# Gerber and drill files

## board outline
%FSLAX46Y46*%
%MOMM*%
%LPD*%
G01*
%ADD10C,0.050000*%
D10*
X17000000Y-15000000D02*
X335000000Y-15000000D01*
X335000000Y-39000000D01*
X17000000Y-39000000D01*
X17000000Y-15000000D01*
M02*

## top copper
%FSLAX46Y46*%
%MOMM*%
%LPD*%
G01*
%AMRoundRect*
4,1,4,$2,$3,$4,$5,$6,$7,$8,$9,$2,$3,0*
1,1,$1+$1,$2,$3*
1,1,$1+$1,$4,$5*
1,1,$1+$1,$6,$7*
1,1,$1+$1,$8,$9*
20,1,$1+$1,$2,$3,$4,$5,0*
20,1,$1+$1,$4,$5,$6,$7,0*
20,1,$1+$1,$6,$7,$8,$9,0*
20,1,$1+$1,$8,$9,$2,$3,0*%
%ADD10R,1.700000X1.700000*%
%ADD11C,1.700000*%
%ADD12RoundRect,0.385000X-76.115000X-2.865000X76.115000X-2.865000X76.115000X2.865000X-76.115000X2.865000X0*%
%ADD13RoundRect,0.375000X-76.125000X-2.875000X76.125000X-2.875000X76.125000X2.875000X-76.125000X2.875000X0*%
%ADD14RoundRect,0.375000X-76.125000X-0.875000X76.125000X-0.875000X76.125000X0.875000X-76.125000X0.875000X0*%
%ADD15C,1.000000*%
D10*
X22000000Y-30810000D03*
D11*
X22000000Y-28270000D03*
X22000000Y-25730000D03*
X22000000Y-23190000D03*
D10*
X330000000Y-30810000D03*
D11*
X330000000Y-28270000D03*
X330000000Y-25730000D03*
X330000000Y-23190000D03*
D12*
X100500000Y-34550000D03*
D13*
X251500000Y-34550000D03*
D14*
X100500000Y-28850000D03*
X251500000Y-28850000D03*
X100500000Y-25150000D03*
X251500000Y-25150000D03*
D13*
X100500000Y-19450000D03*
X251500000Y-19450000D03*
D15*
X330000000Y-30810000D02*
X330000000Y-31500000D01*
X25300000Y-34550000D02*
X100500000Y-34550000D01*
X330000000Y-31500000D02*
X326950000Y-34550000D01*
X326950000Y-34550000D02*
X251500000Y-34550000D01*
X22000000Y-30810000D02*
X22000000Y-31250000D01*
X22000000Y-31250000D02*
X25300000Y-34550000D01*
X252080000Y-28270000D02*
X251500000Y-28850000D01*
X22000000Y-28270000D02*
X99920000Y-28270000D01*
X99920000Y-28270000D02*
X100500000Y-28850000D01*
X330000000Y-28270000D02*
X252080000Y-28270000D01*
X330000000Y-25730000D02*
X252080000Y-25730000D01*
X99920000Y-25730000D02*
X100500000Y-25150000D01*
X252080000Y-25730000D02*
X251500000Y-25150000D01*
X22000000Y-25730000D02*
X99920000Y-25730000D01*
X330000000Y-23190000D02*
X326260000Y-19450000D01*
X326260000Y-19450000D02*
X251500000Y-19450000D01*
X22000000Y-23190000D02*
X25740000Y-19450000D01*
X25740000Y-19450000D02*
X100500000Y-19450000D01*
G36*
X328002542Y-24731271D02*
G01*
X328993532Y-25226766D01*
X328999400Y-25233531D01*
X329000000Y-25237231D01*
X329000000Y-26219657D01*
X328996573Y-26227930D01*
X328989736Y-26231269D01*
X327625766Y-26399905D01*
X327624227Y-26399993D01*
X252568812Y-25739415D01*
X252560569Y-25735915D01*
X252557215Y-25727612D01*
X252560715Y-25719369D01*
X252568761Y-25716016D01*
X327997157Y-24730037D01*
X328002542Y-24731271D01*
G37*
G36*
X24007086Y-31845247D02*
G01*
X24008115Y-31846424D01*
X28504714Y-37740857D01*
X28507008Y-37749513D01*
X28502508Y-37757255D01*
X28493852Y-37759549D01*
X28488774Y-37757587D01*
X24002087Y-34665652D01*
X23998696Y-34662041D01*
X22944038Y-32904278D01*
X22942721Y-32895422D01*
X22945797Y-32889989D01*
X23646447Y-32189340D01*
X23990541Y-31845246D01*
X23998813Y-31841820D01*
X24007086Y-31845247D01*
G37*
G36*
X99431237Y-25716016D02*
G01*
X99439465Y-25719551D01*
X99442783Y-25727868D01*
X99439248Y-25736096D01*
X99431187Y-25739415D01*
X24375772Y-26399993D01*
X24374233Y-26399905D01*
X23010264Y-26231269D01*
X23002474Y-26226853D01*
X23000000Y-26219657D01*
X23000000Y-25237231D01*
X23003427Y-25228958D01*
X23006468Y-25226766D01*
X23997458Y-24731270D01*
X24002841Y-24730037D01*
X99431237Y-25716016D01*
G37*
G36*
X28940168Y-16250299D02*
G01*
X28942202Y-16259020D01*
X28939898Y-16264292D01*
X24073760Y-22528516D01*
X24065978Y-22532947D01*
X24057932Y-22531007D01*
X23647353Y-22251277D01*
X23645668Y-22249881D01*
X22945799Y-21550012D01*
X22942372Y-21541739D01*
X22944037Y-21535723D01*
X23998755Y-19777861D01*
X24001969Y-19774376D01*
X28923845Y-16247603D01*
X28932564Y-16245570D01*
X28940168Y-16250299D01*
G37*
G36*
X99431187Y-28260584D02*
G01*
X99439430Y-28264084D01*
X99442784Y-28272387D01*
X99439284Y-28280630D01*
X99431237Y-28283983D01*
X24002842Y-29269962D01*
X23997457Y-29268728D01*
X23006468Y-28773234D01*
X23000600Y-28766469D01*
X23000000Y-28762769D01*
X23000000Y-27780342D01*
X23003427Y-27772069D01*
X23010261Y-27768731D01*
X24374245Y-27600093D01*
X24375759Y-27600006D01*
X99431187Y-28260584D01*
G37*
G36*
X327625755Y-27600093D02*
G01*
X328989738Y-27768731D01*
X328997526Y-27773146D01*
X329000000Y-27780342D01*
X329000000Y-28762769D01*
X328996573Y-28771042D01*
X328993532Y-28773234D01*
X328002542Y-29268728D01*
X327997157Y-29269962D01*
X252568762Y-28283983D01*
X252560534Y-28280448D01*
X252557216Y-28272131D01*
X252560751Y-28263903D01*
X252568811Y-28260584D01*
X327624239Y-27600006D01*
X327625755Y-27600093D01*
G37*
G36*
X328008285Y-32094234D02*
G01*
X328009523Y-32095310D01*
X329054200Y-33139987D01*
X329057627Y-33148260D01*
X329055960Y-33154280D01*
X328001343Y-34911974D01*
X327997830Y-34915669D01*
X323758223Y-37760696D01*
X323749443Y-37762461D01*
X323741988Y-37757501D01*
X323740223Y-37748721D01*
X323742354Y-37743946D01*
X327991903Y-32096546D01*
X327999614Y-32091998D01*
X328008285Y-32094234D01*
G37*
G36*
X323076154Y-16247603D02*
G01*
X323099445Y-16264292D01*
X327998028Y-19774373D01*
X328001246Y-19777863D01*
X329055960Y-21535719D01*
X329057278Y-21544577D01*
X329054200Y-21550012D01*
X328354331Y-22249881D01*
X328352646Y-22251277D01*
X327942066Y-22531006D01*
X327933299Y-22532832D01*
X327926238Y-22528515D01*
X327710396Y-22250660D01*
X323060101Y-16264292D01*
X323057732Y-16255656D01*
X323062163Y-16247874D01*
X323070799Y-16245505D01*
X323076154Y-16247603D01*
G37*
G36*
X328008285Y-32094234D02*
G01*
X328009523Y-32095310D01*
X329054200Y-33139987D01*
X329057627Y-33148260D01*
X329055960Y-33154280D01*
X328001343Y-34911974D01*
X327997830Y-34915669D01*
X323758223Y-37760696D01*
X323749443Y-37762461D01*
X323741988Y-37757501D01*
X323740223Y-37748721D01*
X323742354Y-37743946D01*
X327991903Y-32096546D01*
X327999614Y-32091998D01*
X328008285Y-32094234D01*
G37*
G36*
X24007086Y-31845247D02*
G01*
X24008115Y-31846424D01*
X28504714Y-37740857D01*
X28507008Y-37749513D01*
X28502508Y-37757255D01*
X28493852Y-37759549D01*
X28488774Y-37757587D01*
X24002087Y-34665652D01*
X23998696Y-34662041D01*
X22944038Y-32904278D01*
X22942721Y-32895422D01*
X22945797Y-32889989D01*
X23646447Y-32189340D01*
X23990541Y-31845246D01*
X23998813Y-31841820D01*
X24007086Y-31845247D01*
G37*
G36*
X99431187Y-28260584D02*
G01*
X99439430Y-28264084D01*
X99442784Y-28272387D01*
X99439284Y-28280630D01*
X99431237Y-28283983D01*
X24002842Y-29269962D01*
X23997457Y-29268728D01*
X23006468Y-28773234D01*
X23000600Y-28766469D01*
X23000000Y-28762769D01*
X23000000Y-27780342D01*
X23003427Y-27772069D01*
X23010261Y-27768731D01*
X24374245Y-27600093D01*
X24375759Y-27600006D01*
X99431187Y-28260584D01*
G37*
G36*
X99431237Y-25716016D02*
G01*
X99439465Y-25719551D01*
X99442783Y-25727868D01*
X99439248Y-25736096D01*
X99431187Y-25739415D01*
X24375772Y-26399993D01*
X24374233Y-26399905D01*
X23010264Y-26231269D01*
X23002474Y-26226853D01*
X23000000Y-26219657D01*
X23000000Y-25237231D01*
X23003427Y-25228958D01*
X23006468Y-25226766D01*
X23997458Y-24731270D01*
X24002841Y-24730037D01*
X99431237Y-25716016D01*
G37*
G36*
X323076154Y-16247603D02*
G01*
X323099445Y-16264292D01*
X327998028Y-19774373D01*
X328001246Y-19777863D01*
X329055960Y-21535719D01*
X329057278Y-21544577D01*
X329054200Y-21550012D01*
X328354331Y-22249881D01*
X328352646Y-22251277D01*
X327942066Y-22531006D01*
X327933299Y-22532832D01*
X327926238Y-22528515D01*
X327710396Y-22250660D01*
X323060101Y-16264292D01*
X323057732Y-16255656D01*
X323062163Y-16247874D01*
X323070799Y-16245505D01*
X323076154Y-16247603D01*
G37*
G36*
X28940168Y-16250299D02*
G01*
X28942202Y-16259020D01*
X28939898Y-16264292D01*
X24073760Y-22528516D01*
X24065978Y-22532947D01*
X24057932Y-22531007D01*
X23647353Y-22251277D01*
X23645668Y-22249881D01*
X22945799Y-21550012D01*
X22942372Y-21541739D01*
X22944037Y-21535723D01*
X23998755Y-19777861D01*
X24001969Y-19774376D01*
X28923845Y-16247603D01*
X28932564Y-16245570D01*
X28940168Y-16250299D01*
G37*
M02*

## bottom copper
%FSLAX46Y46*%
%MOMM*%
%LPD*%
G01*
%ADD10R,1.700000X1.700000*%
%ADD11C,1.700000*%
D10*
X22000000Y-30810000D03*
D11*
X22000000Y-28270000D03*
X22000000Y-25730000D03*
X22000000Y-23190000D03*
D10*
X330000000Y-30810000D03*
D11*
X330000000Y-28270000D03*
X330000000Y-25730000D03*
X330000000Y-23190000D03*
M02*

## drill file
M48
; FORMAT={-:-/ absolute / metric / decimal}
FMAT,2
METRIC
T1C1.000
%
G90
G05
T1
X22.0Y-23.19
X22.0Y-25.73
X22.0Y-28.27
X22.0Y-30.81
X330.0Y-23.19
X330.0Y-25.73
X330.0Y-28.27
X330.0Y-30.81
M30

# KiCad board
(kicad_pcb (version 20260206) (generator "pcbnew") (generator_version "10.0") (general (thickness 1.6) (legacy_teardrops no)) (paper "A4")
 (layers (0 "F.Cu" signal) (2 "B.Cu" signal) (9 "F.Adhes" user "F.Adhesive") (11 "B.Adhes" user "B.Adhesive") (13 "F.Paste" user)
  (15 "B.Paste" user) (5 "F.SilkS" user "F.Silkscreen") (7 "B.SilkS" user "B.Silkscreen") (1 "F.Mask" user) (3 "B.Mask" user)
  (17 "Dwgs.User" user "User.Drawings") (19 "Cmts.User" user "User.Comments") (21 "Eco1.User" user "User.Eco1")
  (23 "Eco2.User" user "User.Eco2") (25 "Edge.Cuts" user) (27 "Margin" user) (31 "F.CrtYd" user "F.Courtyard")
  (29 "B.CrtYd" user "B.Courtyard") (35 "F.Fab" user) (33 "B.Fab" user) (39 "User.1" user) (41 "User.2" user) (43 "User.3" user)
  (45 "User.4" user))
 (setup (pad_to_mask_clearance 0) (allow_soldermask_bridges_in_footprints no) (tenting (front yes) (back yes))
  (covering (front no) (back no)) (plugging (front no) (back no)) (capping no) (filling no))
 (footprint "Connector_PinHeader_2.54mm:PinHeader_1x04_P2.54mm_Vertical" (layer "F.Cu") (at 22 30.81 180)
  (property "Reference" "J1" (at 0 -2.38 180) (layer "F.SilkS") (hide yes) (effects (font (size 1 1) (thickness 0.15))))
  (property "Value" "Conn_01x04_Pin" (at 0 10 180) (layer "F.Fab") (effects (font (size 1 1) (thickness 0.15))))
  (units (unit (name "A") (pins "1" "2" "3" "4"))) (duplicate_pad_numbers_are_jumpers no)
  (pad "1" thru_hole rect (at 0 0 180) (size 1.7 1.7) (drill 1) (layers "*.Cu" "*.Mask") (remove_unused_layers no) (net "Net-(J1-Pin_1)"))
  (pad "2" thru_hole circle (at 0 2.54 180) (size 1.7 1.7) (drill 1) (layers "*.Cu" "*.Mask") (remove_unused_layers no)
   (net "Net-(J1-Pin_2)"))
  (pad "3" thru_hole circle (at 0 5.08 180) (size 1.7 1.7) (drill 1) (layers "*.Cu" "*.Mask") (remove_unused_layers no)
   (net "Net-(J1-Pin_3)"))
  (pad "4" thru_hole circle (at 0 7.62 180) (size 1.7 1.7) (drill 1) (layers "*.Cu" "*.Mask") (remove_unused_layers no)
   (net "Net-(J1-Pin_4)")))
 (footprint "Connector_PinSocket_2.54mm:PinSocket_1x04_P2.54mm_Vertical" (layer "F.Cu") (at 330 30.81 180)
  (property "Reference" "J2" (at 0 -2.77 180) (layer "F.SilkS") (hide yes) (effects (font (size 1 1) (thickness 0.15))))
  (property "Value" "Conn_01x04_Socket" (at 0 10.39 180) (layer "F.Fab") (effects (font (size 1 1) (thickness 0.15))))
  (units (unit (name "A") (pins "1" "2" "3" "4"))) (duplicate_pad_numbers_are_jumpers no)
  (pad "1" thru_hole rect (at 0 0 180) (size 1.7 1.7) (drill 1) (layers "*.Cu" "*.Mask") (remove_unused_layers no) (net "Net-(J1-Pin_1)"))
  (pad "2" thru_hole circle (at 0 2.54 180) (size 1.7 1.7) (drill 1) (layers "*.Cu" "*.Mask") (remove_unused_layers no)
   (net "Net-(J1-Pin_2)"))
  (pad "3" thru_hole circle (at 0 5.08 180) (size 1.7 1.7) (drill 1) (layers "*.Cu" "*.Mask") (remove_unused_layers no)
   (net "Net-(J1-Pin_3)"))
  (pad "4" thru_hole circle (at 0 7.62 180) (size 1.7 1.7) (drill 1) (layers "*.Cu" "*.Mask") (remove_unused_layers no)
   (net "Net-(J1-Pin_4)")))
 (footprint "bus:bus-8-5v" (layer "F.Cu") (at 23 15)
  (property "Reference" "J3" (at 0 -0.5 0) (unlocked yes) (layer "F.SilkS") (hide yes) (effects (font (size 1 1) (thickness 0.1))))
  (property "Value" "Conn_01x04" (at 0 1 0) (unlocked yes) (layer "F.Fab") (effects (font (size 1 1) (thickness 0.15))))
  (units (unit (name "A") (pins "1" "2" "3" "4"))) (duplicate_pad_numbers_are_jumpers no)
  (pad "1" smd roundrect (at 77.5 19.55) (size 153 6.5) (layers "F.Cu" "F.Mask" "F.Paste") (roundrect_rratio 0.05923076923)
   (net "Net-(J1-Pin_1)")
   (teardrops (best_length_ratio 0.5) (max_length 1) (best_width_ratio 1) (max_width 2) (curved_edges no) (filter_ratio 0.9) (enabled yes)
    (allow_two_segments yes) (prefer_zone_connections yes)))
  (pad "1" smd roundrect (at 228.5 19.55) (size 153 6.5) (layers "F.Cu" "F.Mask" "F.Paste") (roundrect_rratio 0.05769230769)
   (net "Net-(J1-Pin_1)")
   (teardrops (best_length_ratio 0.5) (max_length 1) (best_width_ratio 1) (max_width 2) (curved_edges no) (filter_ratio 0.9) (enabled yes)
    (allow_two_segments yes) (prefer_zone_connections yes)))
  (pad "2" smd roundrect (at 77.5 13.85) (size 153 2.5) (layers "F.Cu" "F.Mask" "F.Paste") (roundrect_rratio 0.15) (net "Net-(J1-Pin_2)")
   (teardrops (best_length_ratio 0.5) (max_length 1) (best_width_ratio 1) (max_width 2) (curved_edges no) (filter_ratio 0.9) (enabled yes)
    (allow_two_segments yes) (prefer_zone_connections yes)))
  (pad "2" smd roundrect (at 228.5 13.85) (size 153 2.5) (layers "F.Cu" "F.Mask" "F.Paste") (roundrect_rratio 0.15) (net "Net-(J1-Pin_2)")
   (teardrops (best_length_ratio 0.5) (max_length 1) (best_width_ratio 1) (max_width 2) (curved_edges no) (filter_ratio 0.9) (enabled yes)
    (allow_two_segments yes) (prefer_zone_connections yes)))
  (pad "3" smd roundrect (at 77.5 10.15) (size 153 2.5) (layers "F.Cu" "F.Mask" "F.Paste") (roundrect_rratio 0.15) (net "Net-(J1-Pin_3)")
   (teardrops (best_length_ratio 0.5) (max_length 1) (best_width_ratio 1) (max_width 2) (curved_edges no) (filter_ratio 0.9) (enabled yes)
    (allow_two_segments yes) (prefer_zone_connections yes)))
  (pad "3" smd roundrect (at 228.5 10.15) (size 153 2.5) (layers "F.Cu" "F.Mask" "F.Paste") (roundrect_rratio 0.15) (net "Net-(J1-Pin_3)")
   (teardrops (best_length_ratio 0.5) (max_length 1) (best_width_ratio 1) (max_width 2) (curved_edges no) (filter_ratio 0.9) (enabled yes)
    (allow_two_segments yes) (prefer_zone_connections yes)))
  (pad "4" smd roundrect (at 77.5 4.45) (size 153 6.5) (layers "F.Cu" "F.Mask" "F.Paste") (roundrect_rratio 0.05769230769)
   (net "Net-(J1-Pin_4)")
   (teardrops (best_length_ratio 0.5) (max_length 1) (best_width_ratio 1) (max_width 2) (curved_edges no) (filter_ratio 0.9) (enabled yes)
    (allow_two_segments yes) (prefer_zone_connections yes)))
  (pad "4" smd roundrect (at 228.5 4.45) (size 153 6.5) (layers "F.Cu" "F.Mask" "F.Paste") (roundrect_rratio 0.05769230769)
   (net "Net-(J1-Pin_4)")
   (teardrops (best_length_ratio 0.5) (max_length 1) (best_width_ratio 1) (max_width 2) (curved_edges no) (filter_ratio 0.9) (enabled yes)
    (allow_two_segments yes) (prefer_zone_connections yes))))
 (gr_rect (start 17 15) (end 335 39) (stroke (width 0.05) (type solid)) (fill no) (layer "Edge.Cuts"))
 (segment (start 330 30.81) (end 330 31.5) (width 1) (layer "F.Cu") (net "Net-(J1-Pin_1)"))
 (segment (start 25.3 34.55) (end 100.5 34.55) (width 1) (layer "F.Cu") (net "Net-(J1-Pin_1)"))
 (segment (start 330 31.5) (end 326.95 34.55) (width 1) (layer "F.Cu") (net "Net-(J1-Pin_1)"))
 (segment (start 326.95 34.55) (end 251.5 34.55) (width 1) (layer "F.Cu") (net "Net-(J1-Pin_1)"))
 (segment (start 22 30.81) (end 22 31.25) (width 1) (layer "F.Cu") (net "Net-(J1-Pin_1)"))
 (segment (start 22 31.25) (end 25.3 34.55) (width 1) (layer "F.Cu") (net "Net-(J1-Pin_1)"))
 (segment (start 252.08 28.27) (end 251.5 28.85) (width 1) (layer "F.Cu") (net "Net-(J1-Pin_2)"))
 (segment (start 22 28.27) (end 99.92 28.27) (width 1) (layer "F.Cu") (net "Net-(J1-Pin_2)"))
 (segment (start 99.92 28.27) (end 100.5 28.85) (width 1) (layer "F.Cu") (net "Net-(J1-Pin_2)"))
 (segment (start 330 28.27) (end 252.08 28.27) (width 1) (layer "F.Cu") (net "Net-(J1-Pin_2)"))
 (segment (start 330 25.73) (end 252.08 25.73) (width 1) (layer "F.Cu") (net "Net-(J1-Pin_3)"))
 (segment (start 99.92 25.73) (end 100.5 25.15) (width 1) (layer "F.Cu") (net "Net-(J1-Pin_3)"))
 (segment (start 252.08 25.73) (end 251.5 25.15) (width 1) (layer "F.Cu") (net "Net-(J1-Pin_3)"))
 (segment (start 22 25.73) (end 99.92 25.73) (width 1) (layer "F.Cu") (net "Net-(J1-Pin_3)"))
 (segment (start 330 23.19) (end 326.26 19.45) (width 1) (layer "F.Cu") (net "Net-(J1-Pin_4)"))
 (segment (start 326.26 19.45) (end 251.5 19.45) (width 1) (layer "F.Cu") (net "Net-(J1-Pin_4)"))
 (segment (start 22 23.19) (end 25.74 19.45) (width 1) (layer "F.Cu") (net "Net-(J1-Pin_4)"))
 (segment (start 25.74 19.45) (end 100.5 19.45) (width 1) (layer "F.Cu") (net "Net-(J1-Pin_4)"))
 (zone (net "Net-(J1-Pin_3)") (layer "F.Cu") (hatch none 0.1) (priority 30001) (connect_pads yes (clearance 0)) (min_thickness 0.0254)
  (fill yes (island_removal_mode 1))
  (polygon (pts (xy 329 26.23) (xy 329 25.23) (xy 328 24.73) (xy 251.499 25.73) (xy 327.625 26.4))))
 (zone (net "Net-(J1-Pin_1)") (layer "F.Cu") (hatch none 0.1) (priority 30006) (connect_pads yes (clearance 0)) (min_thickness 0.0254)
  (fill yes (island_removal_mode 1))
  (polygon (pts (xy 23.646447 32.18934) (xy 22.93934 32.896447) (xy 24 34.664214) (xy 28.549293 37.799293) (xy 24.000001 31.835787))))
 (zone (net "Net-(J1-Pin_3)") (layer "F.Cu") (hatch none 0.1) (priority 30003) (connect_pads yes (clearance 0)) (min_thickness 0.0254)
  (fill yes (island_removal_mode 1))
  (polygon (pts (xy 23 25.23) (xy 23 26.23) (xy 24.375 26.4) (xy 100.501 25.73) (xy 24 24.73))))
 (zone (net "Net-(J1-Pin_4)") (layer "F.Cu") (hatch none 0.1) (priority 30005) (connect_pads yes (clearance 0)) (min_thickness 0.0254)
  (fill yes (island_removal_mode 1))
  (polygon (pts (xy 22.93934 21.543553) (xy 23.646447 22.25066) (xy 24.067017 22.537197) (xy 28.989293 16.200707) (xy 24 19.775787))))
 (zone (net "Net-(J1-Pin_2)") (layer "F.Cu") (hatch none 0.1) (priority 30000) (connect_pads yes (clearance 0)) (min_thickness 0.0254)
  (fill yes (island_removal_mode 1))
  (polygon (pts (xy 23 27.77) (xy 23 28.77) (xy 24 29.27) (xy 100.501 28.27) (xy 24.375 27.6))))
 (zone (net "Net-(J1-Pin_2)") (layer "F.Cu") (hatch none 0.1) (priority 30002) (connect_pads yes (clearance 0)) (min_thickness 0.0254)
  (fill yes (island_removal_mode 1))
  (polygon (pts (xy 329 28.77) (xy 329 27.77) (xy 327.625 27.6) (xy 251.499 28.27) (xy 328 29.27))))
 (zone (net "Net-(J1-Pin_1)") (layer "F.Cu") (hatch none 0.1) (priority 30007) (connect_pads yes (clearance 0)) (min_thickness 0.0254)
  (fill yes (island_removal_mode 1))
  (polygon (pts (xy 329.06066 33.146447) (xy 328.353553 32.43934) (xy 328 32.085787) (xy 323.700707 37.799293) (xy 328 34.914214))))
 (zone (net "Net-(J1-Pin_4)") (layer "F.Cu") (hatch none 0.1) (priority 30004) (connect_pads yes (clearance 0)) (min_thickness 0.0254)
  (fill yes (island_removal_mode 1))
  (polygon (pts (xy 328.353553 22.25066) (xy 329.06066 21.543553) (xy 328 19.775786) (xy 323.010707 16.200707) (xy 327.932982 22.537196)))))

